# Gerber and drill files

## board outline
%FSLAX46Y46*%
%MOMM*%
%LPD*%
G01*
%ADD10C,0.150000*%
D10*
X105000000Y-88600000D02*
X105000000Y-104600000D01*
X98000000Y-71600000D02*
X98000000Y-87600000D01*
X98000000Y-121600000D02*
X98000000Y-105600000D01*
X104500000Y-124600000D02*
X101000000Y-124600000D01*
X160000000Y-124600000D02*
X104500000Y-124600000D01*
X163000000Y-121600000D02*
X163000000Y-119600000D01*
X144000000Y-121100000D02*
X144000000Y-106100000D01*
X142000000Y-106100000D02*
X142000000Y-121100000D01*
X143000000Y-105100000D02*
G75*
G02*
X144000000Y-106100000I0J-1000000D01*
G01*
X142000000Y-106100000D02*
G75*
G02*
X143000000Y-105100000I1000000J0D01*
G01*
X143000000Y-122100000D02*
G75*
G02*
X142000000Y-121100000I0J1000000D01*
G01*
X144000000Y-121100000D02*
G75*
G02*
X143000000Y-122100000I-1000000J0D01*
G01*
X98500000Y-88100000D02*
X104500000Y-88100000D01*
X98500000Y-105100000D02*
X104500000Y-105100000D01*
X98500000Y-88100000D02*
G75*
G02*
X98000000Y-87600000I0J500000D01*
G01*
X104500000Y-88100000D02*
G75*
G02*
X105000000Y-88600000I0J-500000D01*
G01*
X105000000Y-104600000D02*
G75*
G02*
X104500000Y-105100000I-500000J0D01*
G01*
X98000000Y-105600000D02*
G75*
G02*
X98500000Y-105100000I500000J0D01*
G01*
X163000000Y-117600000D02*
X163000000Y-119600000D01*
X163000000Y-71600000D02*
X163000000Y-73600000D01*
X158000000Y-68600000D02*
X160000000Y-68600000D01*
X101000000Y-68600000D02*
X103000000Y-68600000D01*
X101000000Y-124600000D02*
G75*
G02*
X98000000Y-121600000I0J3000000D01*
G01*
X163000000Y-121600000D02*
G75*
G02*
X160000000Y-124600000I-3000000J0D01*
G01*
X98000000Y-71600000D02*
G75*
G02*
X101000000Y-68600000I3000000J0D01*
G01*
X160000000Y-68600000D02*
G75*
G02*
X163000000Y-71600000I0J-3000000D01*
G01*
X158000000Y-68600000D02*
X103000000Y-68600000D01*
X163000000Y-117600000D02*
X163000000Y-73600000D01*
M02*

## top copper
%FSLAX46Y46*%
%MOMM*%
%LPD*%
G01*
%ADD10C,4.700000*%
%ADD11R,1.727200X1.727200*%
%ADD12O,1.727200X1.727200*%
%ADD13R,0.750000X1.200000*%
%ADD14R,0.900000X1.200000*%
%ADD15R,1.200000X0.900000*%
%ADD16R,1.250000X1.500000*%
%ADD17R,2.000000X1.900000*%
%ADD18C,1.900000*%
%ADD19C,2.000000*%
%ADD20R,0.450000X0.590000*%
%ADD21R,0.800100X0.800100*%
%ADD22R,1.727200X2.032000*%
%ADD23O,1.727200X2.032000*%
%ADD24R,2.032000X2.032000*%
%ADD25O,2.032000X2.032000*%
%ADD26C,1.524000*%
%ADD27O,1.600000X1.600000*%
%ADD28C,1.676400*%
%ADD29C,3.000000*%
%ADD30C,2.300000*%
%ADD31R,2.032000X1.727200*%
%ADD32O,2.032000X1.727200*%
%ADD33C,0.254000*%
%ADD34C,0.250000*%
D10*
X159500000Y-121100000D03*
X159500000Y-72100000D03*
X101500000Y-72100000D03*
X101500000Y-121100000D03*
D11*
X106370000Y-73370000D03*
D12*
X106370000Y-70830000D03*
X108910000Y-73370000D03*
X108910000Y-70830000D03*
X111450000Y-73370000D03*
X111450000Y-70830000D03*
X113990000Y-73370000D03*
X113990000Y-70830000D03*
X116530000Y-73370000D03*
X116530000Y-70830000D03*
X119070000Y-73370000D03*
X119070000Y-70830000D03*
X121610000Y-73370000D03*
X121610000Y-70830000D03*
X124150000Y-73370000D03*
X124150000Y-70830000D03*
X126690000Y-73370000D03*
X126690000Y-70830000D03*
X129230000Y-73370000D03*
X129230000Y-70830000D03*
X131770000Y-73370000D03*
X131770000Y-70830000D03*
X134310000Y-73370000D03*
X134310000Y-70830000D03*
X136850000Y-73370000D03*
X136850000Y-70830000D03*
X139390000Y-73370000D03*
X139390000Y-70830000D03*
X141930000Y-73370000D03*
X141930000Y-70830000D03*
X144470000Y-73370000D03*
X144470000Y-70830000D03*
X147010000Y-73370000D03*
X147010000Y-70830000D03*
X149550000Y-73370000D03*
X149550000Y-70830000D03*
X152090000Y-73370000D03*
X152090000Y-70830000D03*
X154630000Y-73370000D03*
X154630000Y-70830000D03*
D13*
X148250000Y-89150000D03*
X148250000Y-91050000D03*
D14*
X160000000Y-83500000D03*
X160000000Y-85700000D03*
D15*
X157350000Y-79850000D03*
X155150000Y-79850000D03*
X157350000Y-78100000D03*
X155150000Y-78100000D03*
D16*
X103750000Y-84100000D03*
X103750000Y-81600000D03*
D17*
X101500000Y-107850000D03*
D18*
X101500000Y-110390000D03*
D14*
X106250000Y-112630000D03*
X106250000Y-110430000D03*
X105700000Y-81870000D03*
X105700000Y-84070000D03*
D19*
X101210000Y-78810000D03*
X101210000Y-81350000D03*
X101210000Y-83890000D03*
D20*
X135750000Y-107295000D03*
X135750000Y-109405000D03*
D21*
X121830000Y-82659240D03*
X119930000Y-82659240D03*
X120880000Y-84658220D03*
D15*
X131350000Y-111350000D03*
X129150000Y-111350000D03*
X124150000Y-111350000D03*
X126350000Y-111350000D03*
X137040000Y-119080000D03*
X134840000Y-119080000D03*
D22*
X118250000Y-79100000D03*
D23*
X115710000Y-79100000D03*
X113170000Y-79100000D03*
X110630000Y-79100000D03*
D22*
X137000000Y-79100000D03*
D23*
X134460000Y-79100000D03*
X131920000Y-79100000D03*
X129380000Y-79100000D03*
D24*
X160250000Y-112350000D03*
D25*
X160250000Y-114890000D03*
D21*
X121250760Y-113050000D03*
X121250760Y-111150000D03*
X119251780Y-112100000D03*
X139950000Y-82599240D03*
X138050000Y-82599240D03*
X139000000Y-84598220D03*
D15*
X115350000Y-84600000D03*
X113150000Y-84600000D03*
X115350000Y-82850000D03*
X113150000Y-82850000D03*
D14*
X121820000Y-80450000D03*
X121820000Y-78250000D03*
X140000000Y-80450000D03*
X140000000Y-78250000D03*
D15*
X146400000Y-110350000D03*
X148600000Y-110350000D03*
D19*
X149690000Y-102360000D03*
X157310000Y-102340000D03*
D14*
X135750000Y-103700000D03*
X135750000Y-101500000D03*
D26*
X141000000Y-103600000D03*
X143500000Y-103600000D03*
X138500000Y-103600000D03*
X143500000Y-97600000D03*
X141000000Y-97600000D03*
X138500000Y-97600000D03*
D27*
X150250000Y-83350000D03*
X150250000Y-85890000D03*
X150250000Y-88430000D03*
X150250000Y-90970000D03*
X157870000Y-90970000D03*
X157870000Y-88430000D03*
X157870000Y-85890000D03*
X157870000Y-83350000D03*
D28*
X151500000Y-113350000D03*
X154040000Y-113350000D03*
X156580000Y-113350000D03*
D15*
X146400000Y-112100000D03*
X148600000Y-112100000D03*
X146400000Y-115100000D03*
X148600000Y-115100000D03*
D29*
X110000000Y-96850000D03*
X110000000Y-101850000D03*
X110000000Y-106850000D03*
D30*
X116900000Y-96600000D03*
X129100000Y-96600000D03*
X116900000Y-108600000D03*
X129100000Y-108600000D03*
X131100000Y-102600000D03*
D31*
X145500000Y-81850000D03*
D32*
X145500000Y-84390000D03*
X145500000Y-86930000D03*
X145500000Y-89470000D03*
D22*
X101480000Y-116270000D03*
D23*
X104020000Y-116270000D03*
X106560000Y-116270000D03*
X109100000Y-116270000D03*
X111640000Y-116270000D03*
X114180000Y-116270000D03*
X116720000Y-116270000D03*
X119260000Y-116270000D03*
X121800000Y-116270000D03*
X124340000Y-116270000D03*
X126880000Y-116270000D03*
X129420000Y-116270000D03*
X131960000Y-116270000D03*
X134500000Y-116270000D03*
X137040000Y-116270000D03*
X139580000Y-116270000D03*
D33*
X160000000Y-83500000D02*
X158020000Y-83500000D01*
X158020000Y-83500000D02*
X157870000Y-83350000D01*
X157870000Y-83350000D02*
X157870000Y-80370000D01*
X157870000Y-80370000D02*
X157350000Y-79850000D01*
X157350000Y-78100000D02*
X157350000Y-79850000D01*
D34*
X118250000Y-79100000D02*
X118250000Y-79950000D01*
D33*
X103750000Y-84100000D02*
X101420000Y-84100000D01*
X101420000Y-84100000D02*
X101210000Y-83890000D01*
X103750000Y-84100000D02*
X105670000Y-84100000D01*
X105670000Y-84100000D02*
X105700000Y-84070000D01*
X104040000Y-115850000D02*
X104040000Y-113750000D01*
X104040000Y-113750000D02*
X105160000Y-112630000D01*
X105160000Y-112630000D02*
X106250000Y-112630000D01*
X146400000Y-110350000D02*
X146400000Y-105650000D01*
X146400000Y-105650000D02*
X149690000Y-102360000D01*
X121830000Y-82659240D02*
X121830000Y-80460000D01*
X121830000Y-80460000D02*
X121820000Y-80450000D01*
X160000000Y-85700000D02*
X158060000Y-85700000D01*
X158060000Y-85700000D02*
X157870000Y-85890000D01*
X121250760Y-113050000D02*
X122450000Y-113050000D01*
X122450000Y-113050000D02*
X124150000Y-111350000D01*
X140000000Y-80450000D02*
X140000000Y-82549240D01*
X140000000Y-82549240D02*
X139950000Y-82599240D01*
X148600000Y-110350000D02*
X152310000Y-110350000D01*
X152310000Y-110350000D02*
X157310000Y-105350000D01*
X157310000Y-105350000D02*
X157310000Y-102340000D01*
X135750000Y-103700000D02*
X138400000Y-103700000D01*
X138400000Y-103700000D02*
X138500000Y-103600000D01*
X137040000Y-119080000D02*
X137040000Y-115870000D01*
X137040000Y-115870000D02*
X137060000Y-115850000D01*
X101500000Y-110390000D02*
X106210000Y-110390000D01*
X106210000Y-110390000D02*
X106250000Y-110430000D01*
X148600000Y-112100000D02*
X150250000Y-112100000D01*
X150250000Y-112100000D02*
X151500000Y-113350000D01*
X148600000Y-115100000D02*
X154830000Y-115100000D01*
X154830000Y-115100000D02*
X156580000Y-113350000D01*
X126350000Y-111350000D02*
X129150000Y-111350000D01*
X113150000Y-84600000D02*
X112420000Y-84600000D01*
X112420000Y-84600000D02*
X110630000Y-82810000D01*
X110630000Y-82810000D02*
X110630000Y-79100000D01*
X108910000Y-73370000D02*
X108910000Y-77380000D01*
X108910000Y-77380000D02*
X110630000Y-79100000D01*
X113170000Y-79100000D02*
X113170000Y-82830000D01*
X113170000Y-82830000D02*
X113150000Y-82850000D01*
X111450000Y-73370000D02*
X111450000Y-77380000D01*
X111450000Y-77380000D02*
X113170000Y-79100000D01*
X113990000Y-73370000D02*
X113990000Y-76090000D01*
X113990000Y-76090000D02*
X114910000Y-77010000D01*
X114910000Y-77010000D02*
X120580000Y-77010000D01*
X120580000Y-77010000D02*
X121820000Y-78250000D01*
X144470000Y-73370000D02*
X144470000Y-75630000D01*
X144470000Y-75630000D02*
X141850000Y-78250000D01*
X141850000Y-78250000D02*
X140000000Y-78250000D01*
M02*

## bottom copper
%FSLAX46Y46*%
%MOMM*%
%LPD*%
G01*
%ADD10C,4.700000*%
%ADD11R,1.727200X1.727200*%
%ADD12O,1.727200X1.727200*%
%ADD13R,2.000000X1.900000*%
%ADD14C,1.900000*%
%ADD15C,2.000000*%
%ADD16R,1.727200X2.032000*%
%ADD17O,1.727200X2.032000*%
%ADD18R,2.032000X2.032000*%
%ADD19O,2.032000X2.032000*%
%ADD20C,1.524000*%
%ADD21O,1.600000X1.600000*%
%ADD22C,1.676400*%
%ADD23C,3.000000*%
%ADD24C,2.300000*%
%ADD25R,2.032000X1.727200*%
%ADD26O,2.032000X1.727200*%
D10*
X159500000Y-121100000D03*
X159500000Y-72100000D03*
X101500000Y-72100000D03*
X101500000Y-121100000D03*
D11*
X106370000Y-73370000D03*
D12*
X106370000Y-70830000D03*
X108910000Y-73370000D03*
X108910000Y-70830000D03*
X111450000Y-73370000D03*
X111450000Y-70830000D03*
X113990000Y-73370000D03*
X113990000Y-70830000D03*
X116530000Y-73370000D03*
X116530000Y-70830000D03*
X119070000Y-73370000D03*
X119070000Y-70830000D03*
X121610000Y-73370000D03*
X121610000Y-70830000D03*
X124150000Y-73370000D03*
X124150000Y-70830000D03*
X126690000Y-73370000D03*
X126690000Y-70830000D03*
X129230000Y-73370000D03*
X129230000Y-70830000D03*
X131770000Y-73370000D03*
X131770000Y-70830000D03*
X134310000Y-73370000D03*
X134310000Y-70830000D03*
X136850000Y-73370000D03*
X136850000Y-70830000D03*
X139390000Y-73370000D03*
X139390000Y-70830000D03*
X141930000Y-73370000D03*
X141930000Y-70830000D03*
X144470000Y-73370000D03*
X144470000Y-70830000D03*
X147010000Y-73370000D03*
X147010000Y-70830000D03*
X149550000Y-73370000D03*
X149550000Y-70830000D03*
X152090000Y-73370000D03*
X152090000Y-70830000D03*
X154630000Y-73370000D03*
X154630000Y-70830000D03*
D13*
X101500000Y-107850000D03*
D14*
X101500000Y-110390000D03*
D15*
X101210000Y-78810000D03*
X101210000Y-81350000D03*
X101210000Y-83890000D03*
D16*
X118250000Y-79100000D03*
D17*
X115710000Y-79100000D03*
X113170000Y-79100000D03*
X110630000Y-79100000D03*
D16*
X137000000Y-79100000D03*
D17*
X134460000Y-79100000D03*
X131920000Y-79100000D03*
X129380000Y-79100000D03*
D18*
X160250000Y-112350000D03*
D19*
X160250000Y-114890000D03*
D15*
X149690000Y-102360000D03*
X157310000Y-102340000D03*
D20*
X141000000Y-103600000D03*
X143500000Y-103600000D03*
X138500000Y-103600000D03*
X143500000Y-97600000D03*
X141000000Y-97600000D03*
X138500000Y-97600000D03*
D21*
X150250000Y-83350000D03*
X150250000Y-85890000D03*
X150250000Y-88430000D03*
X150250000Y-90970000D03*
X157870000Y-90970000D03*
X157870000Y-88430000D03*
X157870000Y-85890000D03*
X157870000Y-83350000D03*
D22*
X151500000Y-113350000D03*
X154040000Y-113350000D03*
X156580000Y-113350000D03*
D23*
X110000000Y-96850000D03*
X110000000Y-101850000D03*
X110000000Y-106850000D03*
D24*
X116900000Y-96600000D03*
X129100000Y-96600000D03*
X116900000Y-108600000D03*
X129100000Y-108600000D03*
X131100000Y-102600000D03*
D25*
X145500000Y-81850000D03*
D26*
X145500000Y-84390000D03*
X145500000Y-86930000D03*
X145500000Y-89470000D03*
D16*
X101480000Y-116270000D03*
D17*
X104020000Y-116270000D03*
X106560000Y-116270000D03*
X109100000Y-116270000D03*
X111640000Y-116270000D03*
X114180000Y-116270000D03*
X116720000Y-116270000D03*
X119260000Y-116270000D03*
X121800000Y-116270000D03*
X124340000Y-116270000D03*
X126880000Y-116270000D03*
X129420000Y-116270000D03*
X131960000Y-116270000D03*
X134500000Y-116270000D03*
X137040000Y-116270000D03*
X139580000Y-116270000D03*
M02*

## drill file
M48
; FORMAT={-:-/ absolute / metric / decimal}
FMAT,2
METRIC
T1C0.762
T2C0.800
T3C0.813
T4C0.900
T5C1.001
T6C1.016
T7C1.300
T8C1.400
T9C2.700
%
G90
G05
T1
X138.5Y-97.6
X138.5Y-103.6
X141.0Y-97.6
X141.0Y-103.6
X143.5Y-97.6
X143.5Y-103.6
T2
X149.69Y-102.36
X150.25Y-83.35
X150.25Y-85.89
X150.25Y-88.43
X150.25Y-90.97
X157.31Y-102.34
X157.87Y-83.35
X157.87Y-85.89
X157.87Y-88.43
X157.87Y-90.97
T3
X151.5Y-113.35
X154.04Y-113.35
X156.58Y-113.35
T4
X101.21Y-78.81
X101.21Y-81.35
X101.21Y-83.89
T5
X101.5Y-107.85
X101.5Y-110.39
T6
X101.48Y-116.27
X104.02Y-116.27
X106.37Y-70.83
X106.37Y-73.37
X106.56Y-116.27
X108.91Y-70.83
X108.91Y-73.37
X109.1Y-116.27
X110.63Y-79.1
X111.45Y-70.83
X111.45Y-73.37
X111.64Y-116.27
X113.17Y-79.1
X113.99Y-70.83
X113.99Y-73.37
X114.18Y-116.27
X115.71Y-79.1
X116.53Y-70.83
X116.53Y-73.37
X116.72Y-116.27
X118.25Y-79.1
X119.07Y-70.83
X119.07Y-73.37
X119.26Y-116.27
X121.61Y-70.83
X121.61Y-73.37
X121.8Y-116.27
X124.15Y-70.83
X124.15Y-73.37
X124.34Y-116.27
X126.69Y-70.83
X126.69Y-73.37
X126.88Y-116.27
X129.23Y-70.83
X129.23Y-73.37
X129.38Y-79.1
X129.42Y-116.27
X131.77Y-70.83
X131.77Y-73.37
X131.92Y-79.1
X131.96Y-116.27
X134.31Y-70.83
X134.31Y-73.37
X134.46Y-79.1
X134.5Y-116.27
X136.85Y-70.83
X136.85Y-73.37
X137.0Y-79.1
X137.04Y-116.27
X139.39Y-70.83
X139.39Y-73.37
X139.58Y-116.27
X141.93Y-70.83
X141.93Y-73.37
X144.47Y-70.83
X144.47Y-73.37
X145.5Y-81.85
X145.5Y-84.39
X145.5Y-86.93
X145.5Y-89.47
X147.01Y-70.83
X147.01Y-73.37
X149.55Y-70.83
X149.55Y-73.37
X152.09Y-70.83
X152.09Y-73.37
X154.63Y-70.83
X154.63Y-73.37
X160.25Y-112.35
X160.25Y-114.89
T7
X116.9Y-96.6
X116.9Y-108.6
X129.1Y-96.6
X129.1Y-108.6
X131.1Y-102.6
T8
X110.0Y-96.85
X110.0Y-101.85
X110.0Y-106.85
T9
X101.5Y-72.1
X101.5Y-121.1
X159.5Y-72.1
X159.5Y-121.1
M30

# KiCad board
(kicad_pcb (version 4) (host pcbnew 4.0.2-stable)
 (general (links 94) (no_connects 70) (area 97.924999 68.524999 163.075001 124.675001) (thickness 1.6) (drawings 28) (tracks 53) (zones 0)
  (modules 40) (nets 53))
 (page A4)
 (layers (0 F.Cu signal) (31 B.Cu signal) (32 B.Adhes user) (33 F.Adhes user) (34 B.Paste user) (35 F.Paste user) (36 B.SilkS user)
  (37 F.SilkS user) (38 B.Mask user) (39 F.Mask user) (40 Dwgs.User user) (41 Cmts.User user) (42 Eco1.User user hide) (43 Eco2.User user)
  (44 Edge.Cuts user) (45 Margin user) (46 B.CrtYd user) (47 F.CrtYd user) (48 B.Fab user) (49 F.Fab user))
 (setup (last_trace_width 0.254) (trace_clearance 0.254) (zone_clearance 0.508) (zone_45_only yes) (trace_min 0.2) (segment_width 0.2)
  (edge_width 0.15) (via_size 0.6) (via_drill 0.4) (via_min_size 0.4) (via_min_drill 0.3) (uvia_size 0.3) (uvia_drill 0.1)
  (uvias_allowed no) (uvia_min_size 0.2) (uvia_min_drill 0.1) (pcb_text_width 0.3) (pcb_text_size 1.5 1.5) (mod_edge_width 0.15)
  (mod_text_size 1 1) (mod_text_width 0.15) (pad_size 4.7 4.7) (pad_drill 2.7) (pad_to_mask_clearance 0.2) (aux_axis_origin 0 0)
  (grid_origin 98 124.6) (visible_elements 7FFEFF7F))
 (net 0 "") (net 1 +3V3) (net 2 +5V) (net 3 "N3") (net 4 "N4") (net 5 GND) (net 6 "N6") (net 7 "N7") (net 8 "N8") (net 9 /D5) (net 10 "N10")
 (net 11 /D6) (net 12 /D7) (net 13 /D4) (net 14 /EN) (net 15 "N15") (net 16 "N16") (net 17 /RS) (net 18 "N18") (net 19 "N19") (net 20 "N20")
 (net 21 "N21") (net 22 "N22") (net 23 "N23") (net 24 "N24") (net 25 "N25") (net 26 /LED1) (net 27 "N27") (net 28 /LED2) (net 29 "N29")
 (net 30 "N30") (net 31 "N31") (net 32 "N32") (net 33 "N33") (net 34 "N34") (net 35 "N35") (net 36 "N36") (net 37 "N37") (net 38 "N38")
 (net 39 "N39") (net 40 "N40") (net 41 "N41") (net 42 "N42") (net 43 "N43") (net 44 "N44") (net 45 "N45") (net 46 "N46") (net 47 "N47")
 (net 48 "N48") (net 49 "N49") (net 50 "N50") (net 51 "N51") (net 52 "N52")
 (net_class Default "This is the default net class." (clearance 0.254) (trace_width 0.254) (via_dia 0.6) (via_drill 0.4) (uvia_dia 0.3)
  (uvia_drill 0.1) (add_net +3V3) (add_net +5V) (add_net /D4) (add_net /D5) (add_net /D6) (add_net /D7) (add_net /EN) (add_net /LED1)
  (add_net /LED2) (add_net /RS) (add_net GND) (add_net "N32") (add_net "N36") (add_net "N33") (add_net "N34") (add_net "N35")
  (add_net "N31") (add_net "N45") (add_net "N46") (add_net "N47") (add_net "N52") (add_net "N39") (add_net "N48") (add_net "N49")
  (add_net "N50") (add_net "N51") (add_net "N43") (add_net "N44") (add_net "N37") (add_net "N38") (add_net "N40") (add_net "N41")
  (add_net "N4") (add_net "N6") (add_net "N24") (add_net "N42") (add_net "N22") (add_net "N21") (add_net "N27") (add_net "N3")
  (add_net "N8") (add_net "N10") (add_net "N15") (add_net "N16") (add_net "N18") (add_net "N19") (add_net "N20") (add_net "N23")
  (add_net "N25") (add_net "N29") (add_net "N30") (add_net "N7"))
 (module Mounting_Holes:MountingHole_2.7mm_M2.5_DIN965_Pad (layer F.Cu) (at 159.5 121.1)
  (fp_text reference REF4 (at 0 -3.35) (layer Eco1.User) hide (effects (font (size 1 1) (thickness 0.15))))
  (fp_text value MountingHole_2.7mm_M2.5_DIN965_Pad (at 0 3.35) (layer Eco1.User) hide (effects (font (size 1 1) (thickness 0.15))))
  (pad 4 thru_hole circle (at 0 0) (size 4.7 4.7) (drill 2.7) (layers *.Cu *.Mask F.SilkS)))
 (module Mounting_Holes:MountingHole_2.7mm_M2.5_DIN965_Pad (layer F.Cu) (at 159.5 72.1)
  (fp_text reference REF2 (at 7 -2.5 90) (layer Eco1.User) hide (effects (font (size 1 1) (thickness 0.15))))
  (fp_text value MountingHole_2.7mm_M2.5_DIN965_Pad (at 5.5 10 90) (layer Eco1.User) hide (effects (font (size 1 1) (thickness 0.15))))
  (pad 2 thru_hole circle (at 0 0) (size 4.7 4.7) (drill 2.7) (layers *.Cu *.Mask F.SilkS)))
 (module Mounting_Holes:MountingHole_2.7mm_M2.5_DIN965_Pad (layer F.Cu) (at 101.5 72.1)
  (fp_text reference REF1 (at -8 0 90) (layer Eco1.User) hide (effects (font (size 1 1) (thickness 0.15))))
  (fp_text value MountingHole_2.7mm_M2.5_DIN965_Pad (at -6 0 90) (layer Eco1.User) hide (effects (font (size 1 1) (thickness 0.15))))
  (pad 1 thru_hole circle (at 0 0) (size 4.7 4.7) (drill 2.7) (layers *.Cu *.Mask F.SilkS)))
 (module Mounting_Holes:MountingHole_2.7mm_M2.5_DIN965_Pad (layer F.Cu) (at 101.5 121.1)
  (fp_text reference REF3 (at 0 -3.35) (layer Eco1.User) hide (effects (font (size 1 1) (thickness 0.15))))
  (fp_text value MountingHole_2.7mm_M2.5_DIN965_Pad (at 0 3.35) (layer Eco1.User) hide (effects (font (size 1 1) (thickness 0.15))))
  (pad 3 thru_hole circle (at 0 0) (size 4.7 4.7) (drill 2.7) (layers *.Cu *.Mask F.SilkS)))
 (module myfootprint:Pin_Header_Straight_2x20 (layer F.Cu) (at 130.5 72.1 90)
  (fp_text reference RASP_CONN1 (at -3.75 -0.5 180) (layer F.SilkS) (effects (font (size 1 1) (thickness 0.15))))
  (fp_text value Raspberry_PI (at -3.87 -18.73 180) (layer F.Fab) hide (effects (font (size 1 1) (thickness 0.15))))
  (pad 1 thru_hole rect (at -1.27 -24.13 90) (size 1.7272 1.7272) (drill 1.016) (layers *.Cu *.Mask F.SilkS) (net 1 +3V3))
  (pad 2 thru_hole oval (at 1.27 -24.13 90) (size 1.7272 1.7272) (drill 1.016) (layers *.Cu *.Mask F.SilkS) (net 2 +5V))
  (pad 3 thru_hole oval (at -1.27 -21.59 90) (size 1.7272 1.7272) (drill 1.016) (layers *.Cu *.Mask F.SilkS) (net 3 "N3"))
  (pad 4 thru_hole oval (at 1.27 -21.59 90) (size 1.7272 1.7272) (drill 1.016) (layers *.Cu *.Mask F.SilkS) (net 2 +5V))
  (pad 5 thru_hole oval (at -1.27 -19.05 90) (size 1.7272 1.7272) (drill 1.016) (layers *.Cu *.Mask F.SilkS) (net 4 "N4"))
  (pad 6 thru_hole oval (at 1.27 -19.05 90) (size 1.7272 1.7272) (drill 1.016) (layers *.Cu *.Mask F.SilkS) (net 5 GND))
  (pad 7 thru_hole oval (at -1.27 -16.51 90) (size 1.7272 1.7272) (drill 1.016) (layers *.Cu *.Mask F.SilkS) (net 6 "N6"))
  (pad 8 thru_hole oval (at 1.27 -16.51 90) (size 1.7272 1.7272) (drill 1.016) (layers *.Cu *.Mask F.SilkS) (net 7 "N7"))
  (pad 9 thru_hole oval (at -1.27 -13.97 90) (size 1.7272 1.7272) (drill 1.016) (layers *.Cu *.Mask F.SilkS) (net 5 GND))
  (pad 10 thru_hole oval (at 1.27 -13.97 90) (size 1.7272 1.7272) (drill 1.016) (layers *.Cu *.Mask F.SilkS) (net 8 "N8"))
  (pad 11 thru_hole oval (at -1.27 -11.43 90) (size 1.7272 1.7272) (drill 1.016) (layers *.Cu *.Mask F.SilkS) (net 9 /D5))
  (pad 12 thru_hole oval (at 1.27 -11.43 90) (size 1.7272 1.7272) (drill 1.016) (layers *.Cu *.Mask F.SilkS) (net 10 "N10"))
  (pad 13 thru_hole oval (at -1.27 -8.89 90) (size 1.7272 1.7272) (drill 1.016) (layers *.Cu *.Mask F.SilkS) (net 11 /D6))
  (pad 14 thru_hole oval (at 1.27 -8.89 90) (size 1.7272 1.7272) (drill 1.016) (layers *.Cu *.Mask F.SilkS) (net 5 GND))
  (pad 15 thru_hole oval (at -1.27 -6.35 90) (size 1.7272 1.7272) (drill 1.016) (layers *.Cu *.Mask F.SilkS) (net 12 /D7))
  (pad 16 thru_hole oval (at 1.27 -6.35 90) (size 1.7272 1.7272) (drill 1.016) (layers *.Cu *.Mask F.SilkS) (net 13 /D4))
  (pad 17 thru_hole oval (at -1.27 -3.81 90) (size 1.7272 1.7272) (drill 1.016) (layers *.Cu *.Mask F.SilkS) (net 1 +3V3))
  (pad 18 thru_hole oval (at 1.27 -3.81 90) (size 1.7272 1.7272) (drill 1.016) (layers *.Cu *.Mask F.SilkS) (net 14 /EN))
  (pad 19 thru_hole oval (at -1.27 -1.27 90) (size 1.7272 1.7272) (drill 1.016) (layers *.Cu *.Mask F.SilkS) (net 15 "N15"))
  (pad 20 thru_hole oval (at 1.27 -1.27 90) (size 1.7272 1.7272) (drill 1.016) (layers *.Cu *.Mask F.SilkS) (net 5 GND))
  (pad 21 thru_hole oval (at -1.27 1.27 90) (size 1.7272 1.7272) (drill 1.016) (layers *.Cu *.Mask F.SilkS) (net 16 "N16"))
  (pad 22 thru_hole oval (at 1.27 1.27 90) (size 1.7272 1.7272) (drill 1.016) (layers *.Cu *.Mask F.SilkS) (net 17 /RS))
  (pad 23 thru_hole oval (at -1.27 3.81 90) (size 1.7272 1.7272) (drill 1.016) (layers *.Cu *.Mask F.SilkS) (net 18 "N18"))
  (pad 24 thru_hole oval (at 1.27 3.81 90) (size 1.7272 1.7272) (drill 1.016) (layers *.Cu *.Mask F.SilkS) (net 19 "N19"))
  (pad 25 thru_hole oval (at -1.27 6.35 90) (size 1.7272 1.7272) (drill 1.016) (layers *.Cu *.Mask F.SilkS) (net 5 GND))
  (pad 26 thru_hole oval (at 1.27 6.35 90) (size 1.7272 1.7272) (drill 1.016) (layers *.Cu *.Mask F.SilkS) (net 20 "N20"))
  (pad 27 thru_hole oval (at -1.27 8.89 90) (size 1.7272 1.7272) (drill 1.016) (layers *.Cu *.Mask F.SilkS) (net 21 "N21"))
  (pad 28 thru_hole oval (at 1.27 8.89 90) (size 1.7272 1.7272) (drill 1.016) (layers *.Cu *.Mask F.SilkS) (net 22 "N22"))
  (pad 29 thru_hole oval (at -1.27 11.43 90) (size 1.7272 1.7272) (drill 1.016) (layers *.Cu *.Mask F.SilkS) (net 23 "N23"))
  (pad 30 thru_hole oval (at 1.27 11.43 90) (size 1.7272 1.7272) (drill 1.016) (layers *.Cu *.Mask F.SilkS) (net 5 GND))
  (pad 31 thru_hole oval (at -1.27 13.97 90) (size 1.7272 1.7272) (drill 1.016) (layers *.Cu *.Mask F.SilkS) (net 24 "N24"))
  (pad 32 thru_hole oval (at 1.27 13.97 90) (size 1.7272 1.7272) (drill 1.016) (layers *.Cu *.Mask F.SilkS) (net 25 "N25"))
  (pad 33 thru_hole oval (at -1.27 16.51 90) (size 1.7272 1.7272) (drill 1.016) (layers *.Cu *.Mask F.SilkS) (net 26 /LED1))
  (pad 34 thru_hole oval (at 1.27 16.51 90) (size 1.7272 1.7272) (drill 1.016) (layers *.Cu *.Mask F.SilkS) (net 5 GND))
  (pad 35 thru_hole oval (at -1.27 19.05 90) (size 1.7272 1.7272) (drill 1.016) (layers *.Cu *.Mask F.SilkS) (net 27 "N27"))
  (pad 36 thru_hole oval (at 1.27 19.05 90) (size 1.7272 1.7272) (drill 1.016) (layers *.Cu *.Mask F.SilkS) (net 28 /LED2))
  (pad 37 thru_hole oval (at -1.27 21.59 90) (size 1.7272 1.7272) (drill 1.016) (layers *.Cu *.Mask F.SilkS) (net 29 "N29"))
  (pad 38 thru_hole oval (at 1.27 21.59 90) (size 1.7272 1.7272) (drill 1.016) (layers *.Cu *.Mask F.SilkS))
  (pad 39 thru_hole oval (at -1.27 24.13 90) (size 1.7272 1.7272) (drill 1.016) (layers *.Cu *.Mask F.SilkS) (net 5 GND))
  (pad 40 thru_hole oval (at 1.27 24.13 90) (size 1.7272 1.7272) (drill 1.016) (layers *.Cu *.Mask F.SilkS) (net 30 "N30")))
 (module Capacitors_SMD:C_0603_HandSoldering (layer F.Cu) (at 148.25 90.1 270)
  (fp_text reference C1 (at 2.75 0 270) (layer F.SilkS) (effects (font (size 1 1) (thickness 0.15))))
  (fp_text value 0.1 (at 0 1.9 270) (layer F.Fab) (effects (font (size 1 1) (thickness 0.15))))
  (pad 1 smd rect (at -0.95 0 270) (size 1.2 0.75) (layers F.Cu F.Paste F.Mask) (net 1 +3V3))
  (pad 2 smd rect (at 0.95 0 270) (size 1.2 0.75) (layers F.Cu F.Paste F.Mask) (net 5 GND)))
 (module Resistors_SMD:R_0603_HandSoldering (layer F.Cu) (at 160 84.6 270)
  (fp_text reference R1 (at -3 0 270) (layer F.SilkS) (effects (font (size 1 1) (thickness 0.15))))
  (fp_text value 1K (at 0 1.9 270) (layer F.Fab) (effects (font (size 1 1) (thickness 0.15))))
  (pad 1 smd rect (at -1.1 0 270) (size 1.2 0.9) (layers F.Cu F.Paste F.Mask) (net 1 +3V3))
  (pad 2 smd rect (at 1.1 0 270) (size 1.2 0.9) (layers F.Cu F.Paste F.Mask) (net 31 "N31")))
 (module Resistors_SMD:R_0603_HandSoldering (layer F.Cu) (at 156.25 79.85 180)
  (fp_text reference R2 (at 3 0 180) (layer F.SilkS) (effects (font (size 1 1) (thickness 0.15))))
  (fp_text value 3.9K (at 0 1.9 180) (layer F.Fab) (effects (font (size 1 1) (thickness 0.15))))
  (pad 1 smd rect (at -1.1 0 180) (size 1.2 0.9) (layers F.Cu F.Paste F.Mask) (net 1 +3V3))
  (pad 2 smd rect (at 1.1 0 180) (size 1.2 0.9) (layers F.Cu F.Paste F.Mask) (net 22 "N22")))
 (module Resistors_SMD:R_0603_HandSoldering (layer F.Cu) (at 156.25 78.1 180)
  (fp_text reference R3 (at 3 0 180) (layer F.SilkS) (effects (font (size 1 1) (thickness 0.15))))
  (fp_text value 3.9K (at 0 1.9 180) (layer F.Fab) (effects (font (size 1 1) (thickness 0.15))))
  (pad 1 smd rect (at -1.1 0 180) (size 1.2 0.9) (layers F.Cu F.Paste F.Mask) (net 1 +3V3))
  (pad 2 smd rect (at 1.1 0 180) (size 1.2 0.9) (layers F.Cu F.Paste F.Mask) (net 21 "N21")))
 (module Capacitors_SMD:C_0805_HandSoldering (layer F.Cu) (at 103.75 82.85 90)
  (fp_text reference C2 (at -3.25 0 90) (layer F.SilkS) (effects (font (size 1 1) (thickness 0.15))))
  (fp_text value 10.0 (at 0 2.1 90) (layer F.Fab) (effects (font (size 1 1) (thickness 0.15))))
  (pad 1 smd rect (at -1.25 0 90) (size 1.5 1.25) (layers F.Cu F.Paste F.Mask) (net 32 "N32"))
  (pad 2 smd rect (at 1.25 0 90) (size 1.5 1.25) (layers F.Cu F.Paste F.Mask) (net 5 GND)))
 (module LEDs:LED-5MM (layer F.Cu) (at 101.5 107.85 270)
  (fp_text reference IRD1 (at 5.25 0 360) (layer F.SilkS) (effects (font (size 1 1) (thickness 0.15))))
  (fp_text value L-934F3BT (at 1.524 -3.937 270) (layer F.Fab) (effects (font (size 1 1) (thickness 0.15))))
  (pad 1 thru_hole rect (at 0 0) (size 2 1.9) (drill 1.00076) (layers *.Cu *.Mask F.SilkS) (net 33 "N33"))
  (pad 2 thru_hole circle (at 2.54 0 270) (size 1.9 1.9) (drill 1.00076) (layers *.Cu *.Mask F.SilkS) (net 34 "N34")))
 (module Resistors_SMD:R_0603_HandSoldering (layer F.Cu) (at 106.25 111.53 90)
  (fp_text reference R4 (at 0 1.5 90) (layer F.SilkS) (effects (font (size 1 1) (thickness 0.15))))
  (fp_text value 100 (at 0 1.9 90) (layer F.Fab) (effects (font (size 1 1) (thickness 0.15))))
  (pad 1 smd rect (at -1.1 0 90) (size 1.2 0.9) (layers F.Cu F.Paste F.Mask) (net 2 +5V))
  (pad 2 smd rect (at 1.1 0 90) (size 1.2 0.9) (layers F.Cu F.Paste F.Mask) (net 34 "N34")))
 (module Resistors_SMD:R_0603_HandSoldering (layer F.Cu) (at 105.7 82.97 270)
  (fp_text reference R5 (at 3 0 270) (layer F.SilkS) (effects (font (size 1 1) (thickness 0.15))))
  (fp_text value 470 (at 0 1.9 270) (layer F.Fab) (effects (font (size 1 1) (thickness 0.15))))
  (pad 1 smd rect (at -1.1 0 270) (size 1.2 0.9) (layers F.Cu F.Paste F.Mask) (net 1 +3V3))
  (pad 2 smd rect (at 1.1 0 270) (size 1.2 0.9) (layers F.Cu F.Paste F.Mask) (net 32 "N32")))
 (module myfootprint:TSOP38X (layer F.Cu) (at 103.75 81.35 270)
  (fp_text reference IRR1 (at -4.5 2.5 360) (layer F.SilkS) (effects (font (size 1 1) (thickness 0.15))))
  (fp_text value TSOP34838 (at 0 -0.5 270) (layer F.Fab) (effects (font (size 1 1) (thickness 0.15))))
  (pad 1 thru_hole circle (at -2.54 2.54 270) (size 2 2) (drill 0.9) (layers *.Cu *.Mask F.SilkS) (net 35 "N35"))
  (pad 2 thru_hole circle (at 0 2.54 270) (size 2 2) (drill 0.9) (layers *.Cu *.Mask F.SilkS) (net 5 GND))
  (pad 3 thru_hole circle (at 2.54 2.54 270) (size 2 2) (drill 0.9) (layers *.Cu *.Mask F.SilkS) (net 32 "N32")))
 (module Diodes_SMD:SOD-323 (layer F.Cu) (at 135.75 108.35 270)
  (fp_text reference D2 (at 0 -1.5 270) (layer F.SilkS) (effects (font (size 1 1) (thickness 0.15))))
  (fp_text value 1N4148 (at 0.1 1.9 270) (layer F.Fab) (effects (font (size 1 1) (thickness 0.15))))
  (pad 1 smd rect (at -1.055 0 270) (size 0.59 0.45) (layers F.Cu F.Paste F.Mask) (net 2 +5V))
  (pad 2 smd rect (at 1.055 0 270) (size 0.59 0.45) (layers F.Cu F.Paste F.Mask) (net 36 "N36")))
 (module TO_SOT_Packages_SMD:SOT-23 (layer F.Cu) (at 120.88 83.66 180)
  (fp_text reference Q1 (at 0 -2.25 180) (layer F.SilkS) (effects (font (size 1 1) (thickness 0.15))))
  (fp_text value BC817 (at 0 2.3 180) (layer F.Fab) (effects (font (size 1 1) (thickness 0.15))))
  (pad 1 smd rect (at -0.95 1.00076 180) (size 0.8001 0.8001) (layers F.Cu F.Paste F.Mask) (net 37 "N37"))
  (pad 2 smd rect (at 0.95 1.00076 180) (size 0.8001 0.8001) (layers F.Cu F.Paste F.Mask) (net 5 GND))
  (pad 3 smd rect (at 0 -0.99822 180) (size 0.8001 0.8001) (layers F.Cu F.Paste F.Mask) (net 33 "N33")))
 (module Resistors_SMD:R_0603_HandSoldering (layer F.Cu) (at 130.25 111.35 180)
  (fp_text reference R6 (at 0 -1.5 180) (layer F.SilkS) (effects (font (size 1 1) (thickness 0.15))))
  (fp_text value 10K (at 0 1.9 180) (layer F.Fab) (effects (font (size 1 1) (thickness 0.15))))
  (pad 1 smd rect (at -1.1 0 180) (size 1.2 0.9) (layers F.Cu F.Paste F.Mask) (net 5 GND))
  (pad 2 smd rect (at 1.1 0 180) (size 1.2 0.9) (layers F.Cu F.Paste F.Mask) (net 27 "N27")))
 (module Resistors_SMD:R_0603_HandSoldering (layer F.Cu) (at 125.25 111.35)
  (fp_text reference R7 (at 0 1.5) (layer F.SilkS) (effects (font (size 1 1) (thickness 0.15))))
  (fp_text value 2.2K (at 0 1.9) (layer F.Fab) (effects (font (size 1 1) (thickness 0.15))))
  (pad 1 smd rect (at -1.1 0) (size 1.2 0.9) (layers F.Cu F.Paste F.Mask) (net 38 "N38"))
  (pad 2 smd rect (at 1.1 0) (size 1.2 0.9) (layers F.Cu F.Paste F.Mask) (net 27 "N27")))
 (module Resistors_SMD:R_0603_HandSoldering (layer F.Cu) (at 135.94 119.08 180)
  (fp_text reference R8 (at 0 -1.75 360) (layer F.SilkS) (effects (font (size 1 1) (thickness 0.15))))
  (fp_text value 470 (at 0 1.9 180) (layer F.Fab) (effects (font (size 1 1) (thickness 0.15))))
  (pad 1 smd rect (at -1.1 0 180) (size 1.2 0.9) (layers F.Cu F.Paste F.Mask) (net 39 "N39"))
  (pad 2 smd rect (at 1.1 0 180) (size 1.2 0.9) (layers F.Cu F.Paste F.Mask) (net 2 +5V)))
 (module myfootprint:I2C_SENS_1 (layer F.Cu) (at 123.5 76.6 270)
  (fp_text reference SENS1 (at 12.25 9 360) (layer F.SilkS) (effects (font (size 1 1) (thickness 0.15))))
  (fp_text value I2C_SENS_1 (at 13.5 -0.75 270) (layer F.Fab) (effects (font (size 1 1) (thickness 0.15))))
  (pad 1 thru_hole rect (at 2.5 5.25 270) (size 2.032 1.7272) (drill 1.016) (layers *.Cu *.Mask F.SilkS) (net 1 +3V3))
  (pad 2 thru_hole oval (at 2.5 7.79 270) (size 2.032 1.7272) (drill 1.016) (layers *.Cu *.Mask F.SilkS) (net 5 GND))
  (pad 3 thru_hole oval (at 2.5 10.33 270) (size 2.032 1.7272) (drill 1.016) (layers *.Cu *.Mask F.SilkS) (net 4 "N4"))
  (pad 4 thru_hole oval (at 2.5 12.87 270) (size 2.032 1.7272) (drill 1.016) (layers *.Cu *.Mask F.SilkS) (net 3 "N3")))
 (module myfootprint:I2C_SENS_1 (layer F.Cu) (at 142.25 76.6 270)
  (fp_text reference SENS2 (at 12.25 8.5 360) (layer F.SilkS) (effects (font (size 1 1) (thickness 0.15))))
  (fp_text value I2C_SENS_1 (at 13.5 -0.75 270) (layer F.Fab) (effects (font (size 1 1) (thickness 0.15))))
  (pad 1 thru_hole rect (at 2.5 5.25 270) (size 2.032 1.7272) (drill 1.016) (layers *.Cu *.Mask F.SilkS) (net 1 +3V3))
  (pad 2 thru_hole oval (at 2.5 7.79 270) (size 2.032 1.7272) (drill 1.016) (layers *.Cu *.Mask F.SilkS) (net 5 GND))
  (pad 3 thru_hole oval (at 2.5 10.33 270) (size 2.032 1.7272) (drill 1.016) (layers *.Cu *.Mask F.SilkS) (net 4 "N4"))
  (pad 4 thru_hole oval (at 2.5 12.87 270) (size 2.032 1.7272) (drill 1.016) (layers *.Cu *.Mask F.SilkS) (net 3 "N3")))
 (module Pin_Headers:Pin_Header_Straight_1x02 (layer F.Cu) (at 160.25 112.35)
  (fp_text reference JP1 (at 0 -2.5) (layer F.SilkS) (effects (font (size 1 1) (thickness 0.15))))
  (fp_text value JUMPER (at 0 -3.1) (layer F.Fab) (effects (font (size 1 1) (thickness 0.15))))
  (pad 1 thru_hole rect (at 0 0) (size 2.032 2.032) (drill 1.016) (layers *.Cu *.Mask F.SilkS) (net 31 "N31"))
  (pad 2 thru_hole oval (at 0 2.54) (size 2.032 2.032) (drill 1.016) (layers *.Cu *.Mask F.SilkS) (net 5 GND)))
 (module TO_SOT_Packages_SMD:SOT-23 (layer F.Cu) (at 120.25 112.1 90)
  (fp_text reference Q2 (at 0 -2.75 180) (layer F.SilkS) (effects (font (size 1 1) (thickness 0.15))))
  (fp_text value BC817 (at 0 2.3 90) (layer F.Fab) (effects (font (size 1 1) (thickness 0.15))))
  (pad 1 smd rect (at -0.95 1.00076 90) (size 0.8001 0.8001) (layers F.Cu F.Paste F.Mask) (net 38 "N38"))
  (pad 2 smd rect (at 0.95 1.00076 90) (size 0.8001 0.8001) (layers F.Cu F.Paste F.Mask) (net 5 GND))
  (pad 3 smd rect (at 0 -0.99822 90) (size 0.8001 0.8001) (layers F.Cu F.Paste F.Mask) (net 36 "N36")))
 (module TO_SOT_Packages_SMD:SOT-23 (layer F.Cu) (at 139 83.6 180)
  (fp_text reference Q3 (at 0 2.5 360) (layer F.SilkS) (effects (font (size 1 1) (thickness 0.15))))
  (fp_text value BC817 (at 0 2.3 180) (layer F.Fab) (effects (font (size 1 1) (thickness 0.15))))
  (pad 1 smd rect (at -0.95 1.00076 180) (size 0.8001 0.8001) (layers F.Cu F.Paste F.Mask) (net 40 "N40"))
  (pad 2 smd rect (at 0.95 1.00076 180) (size 0.8001 0.8001) (layers F.Cu F.Paste F.Mask) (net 5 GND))
  (pad 3 smd rect (at 0 -0.99822 180) (size 0.8001 0.8001) (layers F.Cu F.Paste F.Mask) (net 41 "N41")))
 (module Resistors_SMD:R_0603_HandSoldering (layer F.Cu) (at 114.25 84.6 180)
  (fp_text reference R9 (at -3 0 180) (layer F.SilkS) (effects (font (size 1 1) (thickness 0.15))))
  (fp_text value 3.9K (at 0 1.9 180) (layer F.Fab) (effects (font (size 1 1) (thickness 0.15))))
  (pad 1 smd rect (at -1.1 0 180) (size 1.2 0.9) (layers F.Cu F.Paste F.Mask) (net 1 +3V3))
  (pad 2 smd rect (at 1.1 0 180) (size 1.2 0.9) (layers F.Cu F.Paste F.Mask) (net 3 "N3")))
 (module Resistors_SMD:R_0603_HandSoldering (layer F.Cu) (at 114.25 82.85 180)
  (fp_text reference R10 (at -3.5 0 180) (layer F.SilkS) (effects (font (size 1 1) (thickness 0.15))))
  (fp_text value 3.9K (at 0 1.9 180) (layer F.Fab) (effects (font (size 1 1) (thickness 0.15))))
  (pad 1 smd rect (at -1.1 0 180) (size 1.2 0.9) (layers F.Cu F.Paste F.Mask) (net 1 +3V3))
  (pad 2 smd rect (at 1.1 0 180) (size 1.2 0.9) (layers F.Cu F.Paste F.Mask) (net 4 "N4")))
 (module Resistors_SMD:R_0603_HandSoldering (layer F.Cu) (at 121.82 79.35 90)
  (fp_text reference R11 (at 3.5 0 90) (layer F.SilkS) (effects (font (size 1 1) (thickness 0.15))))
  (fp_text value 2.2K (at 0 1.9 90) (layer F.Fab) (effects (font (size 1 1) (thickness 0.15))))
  (pad 1 smd rect (at -1.1 0 90) (size 1.2 0.9) (layers F.Cu F.Paste F.Mask) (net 37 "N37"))
  (pad 2 smd rect (at 1.1 0 90) (size 1.2 0.9) (layers F.Cu F.Paste F.Mask) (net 6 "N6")))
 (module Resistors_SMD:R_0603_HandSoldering (layer F.Cu) (at 140 79.35 90)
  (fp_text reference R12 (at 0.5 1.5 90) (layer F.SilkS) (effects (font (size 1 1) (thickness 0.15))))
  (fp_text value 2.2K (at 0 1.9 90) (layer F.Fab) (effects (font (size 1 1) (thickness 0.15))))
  (pad 1 smd rect (at -1.1 0 90) (size 1.2 0.9) (layers F.Cu F.Paste F.Mask) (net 40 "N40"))
  (pad 2 smd rect (at 1.1 0 90) (size 1.2 0.9) (layers F.Cu F.Paste F.Mask) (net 24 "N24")))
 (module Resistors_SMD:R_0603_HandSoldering (layer F.Cu) (at 147.5 110.35)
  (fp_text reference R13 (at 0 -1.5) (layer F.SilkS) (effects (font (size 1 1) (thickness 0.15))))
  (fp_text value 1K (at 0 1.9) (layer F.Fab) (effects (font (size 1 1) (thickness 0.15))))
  (pad 1 smd rect (at -1.1 0) (size 1.2 0.9) (layers F.Cu F.Paste F.Mask) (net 2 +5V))
  (pad 2 smd rect (at 1.1 0) (size 1.2 0.9) (layers F.Cu F.Paste F.Mask) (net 41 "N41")))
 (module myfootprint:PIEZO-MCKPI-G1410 (layer F.Cu) (at 153.5 102.35)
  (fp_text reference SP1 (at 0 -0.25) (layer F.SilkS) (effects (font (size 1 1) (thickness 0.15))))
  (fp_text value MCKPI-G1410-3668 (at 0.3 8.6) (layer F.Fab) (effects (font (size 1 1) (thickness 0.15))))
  (pad 1 thru_hole circle (at -3.81 0.01) (size 2 2) (drill 0.8) (layers *.Cu *.Mask F.SilkS) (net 2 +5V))
  (pad 2 thru_hole circle (at 3.81 -0.01) (size 2 2) (drill 0.8) (layers *.Cu *.Mask F.SilkS) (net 41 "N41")))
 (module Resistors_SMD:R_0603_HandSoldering (layer F.Cu) (at 135.75 102.6 90)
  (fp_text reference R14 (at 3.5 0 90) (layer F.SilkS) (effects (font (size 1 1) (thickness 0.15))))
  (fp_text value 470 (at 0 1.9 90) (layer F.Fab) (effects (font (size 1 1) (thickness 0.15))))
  (pad 1 smd rect (at -1.1 0 90) (size 1.2 0.9) (layers F.Cu F.Paste F.Mask) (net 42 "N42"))
  (pad 2 smd rect (at 1.1 0 90) (size 1.2 0.9) (layers F.Cu F.Paste F.Mask) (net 5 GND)))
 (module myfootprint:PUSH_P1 (layer F.Cu) (at 141 100.6)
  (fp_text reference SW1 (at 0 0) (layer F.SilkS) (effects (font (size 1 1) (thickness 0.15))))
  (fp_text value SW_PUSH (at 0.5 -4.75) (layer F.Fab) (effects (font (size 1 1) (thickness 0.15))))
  (pad 1 thru_hole circle (at 0 3) (size 1.524 1.524) (drill 0.762) (layers *.Cu *.Mask F.SilkS) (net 30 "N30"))
  (pad 3 thru_hole circle (at 2.5 3) (size 1.524 1.524) (drill 0.762) (layers *.Cu *.Mask F.SilkS))
  (pad 2 thru_hole circle (at -2.5 3) (size 1.524 1.524) (drill 0.762) (layers *.Cu *.Mask F.SilkS) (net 42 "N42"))
  (pad 2 thru_hole circle (at 2.5 -3) (size 1.524 1.524) (drill 0.762) (layers *.Cu *.Mask F.SilkS) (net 42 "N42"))
  (pad 1 thru_hole circle (at 0 -3) (size 1.524 1.524) (drill 0.762) (layers *.Cu *.Mask F.SilkS) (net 30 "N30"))
  (pad 3 thru_hole circle (at -2.5 -3) (size 1.524 1.524) (drill 0.762) (layers *.Cu *.Mask F.SilkS)))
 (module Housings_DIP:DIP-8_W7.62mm (layer F.Cu) (at 150.25 83.35)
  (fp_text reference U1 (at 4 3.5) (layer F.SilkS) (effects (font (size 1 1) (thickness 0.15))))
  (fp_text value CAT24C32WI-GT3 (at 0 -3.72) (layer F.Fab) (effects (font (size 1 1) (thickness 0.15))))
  (pad 1 thru_hole oval (at 0 0) (size 1.6 1.6) (drill 0.8) (layers *.Cu *.Mask F.SilkS) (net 5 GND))
  (pad 2 thru_hole oval (at 0 2.54) (size 1.6 1.6) (drill 0.8) (layers *.Cu *.Mask F.SilkS) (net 5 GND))
  (pad 3 thru_hole oval (at 0 5.08) (size 1.6 1.6) (drill 0.8) (layers *.Cu *.Mask F.SilkS) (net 5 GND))
  (pad 4 thru_hole oval (at 0 7.62) (size 1.6 1.6) (drill 0.8) (layers *.Cu *.Mask F.SilkS) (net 5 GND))
  (pad 5 thru_hole oval (at 7.62 7.62) (size 1.6 1.6) (drill 0.8) (layers *.Cu *.Mask F.SilkS) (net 21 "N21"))
  (pad 6 thru_hole oval (at 7.62 5.08) (size 1.6 1.6) (drill 0.8) (layers *.Cu *.Mask F.SilkS) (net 22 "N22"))
  (pad 7 thru_hole oval (at 7.62 2.54) (size 1.6 1.6) (drill 0.8) (layers *.Cu *.Mask F.SilkS) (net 31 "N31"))
  (pad 8 thru_hole oval (at 7.62 0) (size 1.6 1.6) (drill 0.8) (layers *.Cu *.Mask F.SilkS) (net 1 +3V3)))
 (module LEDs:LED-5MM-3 (layer F.Cu) (at 151.5 113.35)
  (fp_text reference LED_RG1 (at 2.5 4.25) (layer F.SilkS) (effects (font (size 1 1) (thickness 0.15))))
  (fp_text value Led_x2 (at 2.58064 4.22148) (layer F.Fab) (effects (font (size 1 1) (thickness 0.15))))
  (pad 1 thru_hole circle (at 0 0 180) (size 1.6764 1.6764) (drill 0.8128) (layers *.Cu *.Mask F.SilkS) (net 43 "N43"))
  (pad 2 thru_hole circle (at 2.54 0 180) (size 1.6764 1.6764) (drill 0.8128) (layers *.Cu *.Mask F.SilkS) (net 5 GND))
  (pad 3 thru_hole circle (at 5.08 0 180) (size 1.6764 1.6764) (drill 0.8128) (layers *.Cu *.Mask F.SilkS) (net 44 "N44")))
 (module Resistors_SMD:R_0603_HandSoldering (layer F.Cu) (at 147.5 112.1)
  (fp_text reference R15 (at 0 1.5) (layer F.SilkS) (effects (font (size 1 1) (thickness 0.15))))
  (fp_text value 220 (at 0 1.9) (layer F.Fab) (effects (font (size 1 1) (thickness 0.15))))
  (pad 1 smd rect (at -1.1 0) (size 1.2 0.9) (layers F.Cu F.Paste F.Mask) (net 28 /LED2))
  (pad 2 smd rect (at 1.1 0) (size 1.2 0.9) (layers F.Cu F.Paste F.Mask) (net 43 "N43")))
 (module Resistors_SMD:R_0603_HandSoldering (layer F.Cu) (at 147.5 115.1)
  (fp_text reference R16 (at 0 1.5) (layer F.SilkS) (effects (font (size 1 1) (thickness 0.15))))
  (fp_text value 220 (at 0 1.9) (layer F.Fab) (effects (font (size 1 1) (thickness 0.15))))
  (pad 1 smd rect (at -1.1 0) (size 1.2 0.9) (layers F.Cu F.Paste F.Mask) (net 26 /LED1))
  (pad 2 smd rect (at 1.1 0) (size 1.2 0.9) (layers F.Cu F.Paste F.Mask) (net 44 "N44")))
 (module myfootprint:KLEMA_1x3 (layer F.Cu) (at 113.5 96.85 270)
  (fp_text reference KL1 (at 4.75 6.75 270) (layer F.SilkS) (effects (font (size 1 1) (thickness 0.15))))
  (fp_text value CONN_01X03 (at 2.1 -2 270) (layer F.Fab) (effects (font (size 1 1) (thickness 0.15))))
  (pad 1 thru_hole circle (at 0 3.5 270) (size 3 3) (drill 1.4) (layers *.Cu *.Mask F.SilkS) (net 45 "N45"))
  (pad 2 thru_hole circle (at 5 3.5 270) (size 3 3) (drill 1.4) (layers *.Cu *.Mask F.SilkS) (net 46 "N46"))
  (pad 3 thru_hole circle (at 10 3.5 270) (size 3 3) (drill 1.4) (layers *.Cu *.Mask F.SilkS) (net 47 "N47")))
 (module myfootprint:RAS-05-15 (layer F.Cu) (at 119 95.1)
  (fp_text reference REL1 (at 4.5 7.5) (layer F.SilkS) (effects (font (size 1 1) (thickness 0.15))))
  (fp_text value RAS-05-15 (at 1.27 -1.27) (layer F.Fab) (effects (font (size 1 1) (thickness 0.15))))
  (pad 1 thru_hole circle (at -2.1 1.5) (size 2.3 2.3) (drill 1.3) (layers *.Cu *.Mask F.SilkS) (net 47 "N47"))
  (pad 2 thru_hole circle (at 10.1 1.5) (size 2.3 2.3) (drill 1.3) (layers *.Cu *.Mask F.SilkS) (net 2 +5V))
  (pad 3 thru_hole circle (at -2.1 13.5) (size 2.3 2.3) (drill 1.3) (layers *.Cu *.Mask F.SilkS) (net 46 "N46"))
  (pad 4 thru_hole circle (at 10.1 13.5) (size 2.3 2.3) (drill 1.3) (layers *.Cu *.Mask F.SilkS) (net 36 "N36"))
  (pad 5 thru_hole circle (at 12.1 7.5) (size 2.3 2.3) (drill 1.3) (layers *.Cu *.Mask F.SilkS) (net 45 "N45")))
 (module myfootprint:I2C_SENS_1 (layer F.Cu) (at 143 76.6)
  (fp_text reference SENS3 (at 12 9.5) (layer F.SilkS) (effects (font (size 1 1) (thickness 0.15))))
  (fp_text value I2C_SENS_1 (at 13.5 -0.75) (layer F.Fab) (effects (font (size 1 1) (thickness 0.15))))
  (pad 1 thru_hole rect (at 2.5 5.25) (size 2.032 1.7272) (drill 1.016) (layers *.Cu *.Mask F.SilkS) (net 1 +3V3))
  (pad 2 thru_hole oval (at 2.5 7.79) (size 2.032 1.7272) (drill 1.016) (layers *.Cu *.Mask F.SilkS) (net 5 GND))
  (pad 3 thru_hole oval (at 2.5 10.33) (size 2.032 1.7272) (drill 1.016) (layers *.Cu *.Mask F.SilkS) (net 4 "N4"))
  (pad 4 thru_hole oval (at 2.5 12.87) (size 2.032 1.7272) (drill 1.016) (layers *.Cu *.Mask F.SilkS) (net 3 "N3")))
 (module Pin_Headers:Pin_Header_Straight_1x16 (layer F.Cu) (at 101.48 116.27 90)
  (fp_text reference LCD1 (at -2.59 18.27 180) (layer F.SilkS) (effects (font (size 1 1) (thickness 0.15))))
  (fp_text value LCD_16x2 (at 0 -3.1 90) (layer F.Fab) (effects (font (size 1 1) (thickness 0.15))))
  (pad 1 thru_hole rect (at 0 0 90) (size 2.032 1.7272) (drill 1.016) (layers *.Cu *.Mask F.SilkS) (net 5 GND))
  (pad 2 thru_hole oval (at 0 2.54 90) (size 2.032 1.7272) (drill 1.016) (layers *.Cu *.Mask F.SilkS) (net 2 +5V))
  (pad 3 thru_hole oval (at 0 5.08 90) (size 2.032 1.7272) (drill 1.016) (layers *.Cu *.Mask F.SilkS) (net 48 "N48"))
  (pad 4 thru_hole oval (at 0 7.62 90) (size 2.032 1.7272) (drill 1.016) (layers *.Cu *.Mask F.SilkS) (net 17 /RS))
  (pad 5 thru_hole oval (at 0 10.16 90) (size 2.032 1.7272) (drill 1.016) (layers *.Cu *.Mask F.SilkS) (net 5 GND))
  (pad 6 thru_hole oval (at 0 12.7 90) (size 2.032 1.7272) (drill 1.016) (layers *.Cu *.Mask F.SilkS) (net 14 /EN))
  (pad 7 thru_hole oval (at 0 15.24 90) (size 2.032 1.7272) (drill 1.016) (layers *.Cu *.Mask F.SilkS) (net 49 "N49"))
  (pad 8 thru_hole oval (at 0 17.78 90) (size 2.032 1.7272) (drill 1.016) (layers *.Cu *.Mask F.SilkS) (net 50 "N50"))
  (pad 9 thru_hole oval (at 0 20.32 90) (size 2.032 1.7272) (drill 1.016) (layers *.Cu *.Mask F.SilkS) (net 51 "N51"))
  (pad 10 thru_hole oval (at 0 22.86 90) (size 2.032 1.7272) (drill 1.016) (layers *.Cu *.Mask F.SilkS) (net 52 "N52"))
  (pad 11 thru_hole oval (at 0 25.4 90) (size 2.032 1.7272) (drill 1.016) (layers *.Cu *.Mask F.SilkS) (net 13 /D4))
  (pad 12 thru_hole oval (at 0 27.94 90) (size 2.032 1.7272) (drill 1.016) (layers *.Cu *.Mask F.SilkS) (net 9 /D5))
  (pad 13 thru_hole oval (at 0 30.48 90) (size 2.032 1.7272) (drill 1.016) (layers *.Cu *.Mask F.SilkS) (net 11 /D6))
  (pad 14 thru_hole oval (at 0 33.02 90) (size 2.032 1.7272) (drill 1.016) (layers *.Cu *.Mask F.SilkS) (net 12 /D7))
  (pad 15 thru_hole oval (at 0 35.56 90) (size 2.032 1.7272) (drill 1.016) (layers *.Cu *.Mask F.SilkS) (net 39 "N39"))
  (pad 16 thru_hole oval (at 0 38.1 90) (size 2.032 1.7272) (drill 1.016) (layers *.Cu *.Mask F.SilkS) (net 5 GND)))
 (gr_line (start 105 88.6) (end 105 104.6) (angle 90) (layer Edge.Cuts) (width 0.15))
 (gr_line (start 98 71.6) (end 98 87.6) (angle 90) (layer Edge.Cuts) (width 0.15))
 (gr_line (start 98 121.6) (end 98 105.6) (angle 90) (layer Edge.Cuts) (width 0.15))
 (gr_line (start 104.5 124.6) (end 101 124.6) (angle 90) (layer Edge.Cuts) (width 0.15))
 (gr_line (start 160 124.6) (end 104.5 124.6) (angle 90) (layer Edge.Cuts) (width 0.15))
 (gr_line (start 163 121.6) (end 163 119.6) (angle 90) (layer Edge.Cuts) (width 0.15))
 (gr_line (start 144 121.1) (end 144 106.1) (angle 90) (layer Edge.Cuts) (width 0.15))
 (gr_line (start 142 106.1) (end 142 121.1) (angle 90) (layer Edge.Cuts) (width 0.15))
 (gr_arc (start 143 106.1) (end 143 105.1) (angle 90) (layer Edge.Cuts) (width 0.15))
 (gr_arc (start 143 106.1) (end 142 106.1) (angle 90) (layer Edge.Cuts) (width 0.15))
 (gr_arc (start 143 121.1) (end 143 122.1) (angle 90) (layer Edge.Cuts) (width 0.15))
 (gr_arc (start 143 121.1) (end 144 121.1) (angle 90) (layer Edge.Cuts) (width 0.15))
 (gr_line (start 98.5 88.1) (end 104.5 88.1) (angle 90) (layer Edge.Cuts) (width 0.15))
 (gr_line (start 98.5 105.1) (end 104.5 105.1) (angle 90) (layer Edge.Cuts) (width 0.15))
 (gr_arc (start 98.5 87.6) (end 98.5 88.1) (angle 90) (layer Edge.Cuts) (width 0.15))
 (gr_arc (start 104.5 88.6) (end 104.5 88.1) (angle 90) (layer Edge.Cuts) (width 0.15))
 (gr_arc (start 104.5 104.6) (end 105 104.6) (angle 90) (layer Edge.Cuts) (width 0.15))
 (gr_arc (start 98.5 105.6) (end 98 105.6) (angle 90) (layer Edge.Cuts) (width 0.15))
 (gr_line (start 163 117.6) (end 163 119.6) (angle 90) (layer Edge.Cuts) (width 0.15))
 (gr_line (start 163 71.6) (end 163 73.6) (angle 90) (layer Edge.Cuts) (width 0.15))
 (gr_line (start 158 68.6) (end 160 68.6) (angle 90) (layer Edge.Cuts) (width 0.15))
 (gr_line (start 101 68.6) (end 103 68.6) (angle 90) (layer Edge.Cuts) (width 0.15))
 (gr_arc (start 101 121.6) (end 101 124.6) (angle 90) (layer Edge.Cuts) (width 0.15))
 (gr_arc (start 160 121.6) (end 163 121.6) (angle 90) (layer Edge.Cuts) (width 0.15))
 (gr_arc (start 101 71.6) (end 98 71.6) (angle 90) (layer Edge.Cuts) (width 0.15))
 (gr_arc (start 160 71.6) (end 160 68.6) (angle 90) (layer Edge.Cuts) (width 0.15))
 (gr_line (start 158 68.6) (end 103 68.6) (angle 90) (layer Edge.Cuts) (width 0.15))
 (gr_line (start 163 117.6) (end 163 73.6) (angle 90) (layer Edge.Cuts) (width 0.15))
 (segment (start 160 83.5) (end 158.02 83.5) (width 0.254) (layer F.Cu) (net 1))
 (segment (start 158.02 83.5) (end 157.87 83.35) (width 0.254) (layer F.Cu) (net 1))
 (segment (start 157.87 83.35) (end 157.87 80.37) (width 0.254) (layer F.Cu) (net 1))
 (segment (start 157.87 80.37) (end 157.35 79.85) (width 0.254) (layer F.Cu) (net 1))
 (segment (start 157.35 78.1) (end 157.35 79.85) (width 0.254) (layer F.Cu) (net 1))
 (segment (start 118.25 79.1) (end 118.25 79.95) (width 0.25) (layer F.Cu) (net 1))
 (segment (start 103.75 84.1) (end 101.42 84.1) (width 0.254) (layer F.Cu) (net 32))
 (segment (start 101.42 84.1) (end 101.21 83.89) (width 0.254) (layer F.Cu) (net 32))
 (segment (start 103.75 84.1) (end 105.67 84.1) (width 0.254) (layer F.Cu) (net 32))
 (segment (start 105.67 84.1) (end 105.7 84.07) (width 0.254) (layer F.Cu) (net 32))
 (segment (start 104.04 115.85) (end 104.04 113.75) (width 0.254) (layer F.Cu) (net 2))
 (segment (start 104.04 113.75) (end 105.16 112.63) (width 0.254) (layer F.Cu) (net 2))
 (segment (start 105.16 112.63) (end 106.25 112.63) (width 0.254) (layer F.Cu) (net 2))
 (segment (start 146.4 110.35) (end 146.4 105.65) (width 0.254) (layer F.Cu) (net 2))
 (segment (start 146.4 105.65) (end 149.69 102.36) (width 0.254) (layer F.Cu) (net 2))
 (segment (start 121.83 82.65924) (end 121.83 80.46) (width 0.254) (layer F.Cu) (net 37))
 (segment (start 121.83 80.46) (end 121.82 80.45) (width 0.254) (layer F.Cu) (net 37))
 (segment (start 160 85.7) (end 158.06 85.7) (width 0.254) (layer F.Cu) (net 31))
 (segment (start 158.06 85.7) (end 157.87 85.89) (width 0.254) (layer F.Cu) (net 31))
 (segment (start 121.25076 113.05) (end 122.45 113.05) (width 0.254) (layer F.Cu) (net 38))
 (segment (start 122.45 113.05) (end 124.15 111.35) (width 0.254) (layer F.Cu) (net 38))
 (segment (start 140 80.45) (end 140 82.54924) (width 0.254) (layer F.Cu) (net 40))
 (segment (start 140 82.54924) (end 139.95 82.59924) (width 0.254) (layer F.Cu) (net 40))
 (segment (start 148.6 110.35) (end 152.31 110.35) (width 0.254) (layer F.Cu) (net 41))
 (segment (start 152.31 110.35) (end 157.31 105.35) (width 0.254) (layer F.Cu) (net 41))
 (segment (start 157.31 105.35) (end 157.31 102.34) (width 0.254) (layer F.Cu) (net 41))
 (segment (start 135.75 103.7) (end 138.4 103.7) (width 0.254) (layer F.Cu) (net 42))
 (segment (start 138.4 103.7) (end 138.5 103.6) (width 0.254) (layer F.Cu) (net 42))
 (segment (start 137.04 119.08) (end 137.04 115.87) (width 0.254) (layer F.Cu) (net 39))
 (segment (start 137.04 115.87) (end 137.06 115.85) (width 0.254) (layer F.Cu) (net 39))
 (segment (start 101.5 110.39) (end 106.21 110.39) (width 0.254) (layer F.Cu) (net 34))
 (segment (start 106.21 110.39) (end 106.25 110.43) (width 0.254) (layer F.Cu) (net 34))
 (segment (start 148.6 112.1) (end 150.25 112.1) (width 0.254) (layer F.Cu) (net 43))
 (segment (start 150.25 112.1) (end 151.5 113.35) (width 0.254) (layer F.Cu) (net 43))
 (segment (start 148.6 115.1) (end 154.83 115.1) (width 0.254) (layer F.Cu) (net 44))
 (segment (start 154.83 115.1) (end 156.58 113.35) (width 0.254) (layer F.Cu) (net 44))
 (segment (start 126.35 111.35) (end 129.15 111.35) (width 0.254) (layer F.Cu) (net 27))
 (segment (start 113.15 84.6) (end 112.42 84.6) (width 0.254) (layer F.Cu) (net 3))
 (segment (start 112.42 84.6) (end 110.63 82.81) (width 0.254) (layer F.Cu) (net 3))
 (segment (start 110.63 82.81) (end 110.63 79.1) (width 0.254) (layer F.Cu) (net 3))
 (segment (start 108.91 73.37) (end 108.91 77.38) (width 0.254) (layer F.Cu) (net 3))
 (segment (start 108.91 77.38) (end 110.63 79.1) (width 0.254) (layer F.Cu) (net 3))
 (segment (start 113.17 79.1) (end 113.17 82.83) (width 0.254) (layer F.Cu) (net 4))
 (segment (start 113.17 82.83) (end 113.15 82.85) (width 0.254) (layer F.Cu) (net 4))
 (segment (start 111.45 73.37) (end 111.45 77.38) (width 0.254) (layer F.Cu) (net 4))
 (segment (start 111.45 77.38) (end 113.17 79.1) (width 0.254) (layer F.Cu) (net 4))
 (segment (start 113.99 73.37) (end 113.99 76.09) (width 0.254) (layer F.Cu) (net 6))
 (segment (start 113.99 76.09) (end 114.91 77.01) (width 0.254) (layer F.Cu) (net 6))
 (segment (start 114.91 77.01) (end 120.58 77.01) (width 0.254) (layer F.Cu) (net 6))
 (segment (start 120.58 77.01) (end 121.82 78.25) (width 0.254) (layer F.Cu) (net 6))
 (segment (start 144.47 73.37) (end 144.47 75.63) (width 0.254) (layer F.Cu) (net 24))
 (segment (start 144.47 75.63) (end 141.85 78.25) (width 0.254) (layer F.Cu) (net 24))
 (segment (start 141.85 78.25) (end 140 78.25) (width 0.254) (layer F.Cu) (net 24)))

